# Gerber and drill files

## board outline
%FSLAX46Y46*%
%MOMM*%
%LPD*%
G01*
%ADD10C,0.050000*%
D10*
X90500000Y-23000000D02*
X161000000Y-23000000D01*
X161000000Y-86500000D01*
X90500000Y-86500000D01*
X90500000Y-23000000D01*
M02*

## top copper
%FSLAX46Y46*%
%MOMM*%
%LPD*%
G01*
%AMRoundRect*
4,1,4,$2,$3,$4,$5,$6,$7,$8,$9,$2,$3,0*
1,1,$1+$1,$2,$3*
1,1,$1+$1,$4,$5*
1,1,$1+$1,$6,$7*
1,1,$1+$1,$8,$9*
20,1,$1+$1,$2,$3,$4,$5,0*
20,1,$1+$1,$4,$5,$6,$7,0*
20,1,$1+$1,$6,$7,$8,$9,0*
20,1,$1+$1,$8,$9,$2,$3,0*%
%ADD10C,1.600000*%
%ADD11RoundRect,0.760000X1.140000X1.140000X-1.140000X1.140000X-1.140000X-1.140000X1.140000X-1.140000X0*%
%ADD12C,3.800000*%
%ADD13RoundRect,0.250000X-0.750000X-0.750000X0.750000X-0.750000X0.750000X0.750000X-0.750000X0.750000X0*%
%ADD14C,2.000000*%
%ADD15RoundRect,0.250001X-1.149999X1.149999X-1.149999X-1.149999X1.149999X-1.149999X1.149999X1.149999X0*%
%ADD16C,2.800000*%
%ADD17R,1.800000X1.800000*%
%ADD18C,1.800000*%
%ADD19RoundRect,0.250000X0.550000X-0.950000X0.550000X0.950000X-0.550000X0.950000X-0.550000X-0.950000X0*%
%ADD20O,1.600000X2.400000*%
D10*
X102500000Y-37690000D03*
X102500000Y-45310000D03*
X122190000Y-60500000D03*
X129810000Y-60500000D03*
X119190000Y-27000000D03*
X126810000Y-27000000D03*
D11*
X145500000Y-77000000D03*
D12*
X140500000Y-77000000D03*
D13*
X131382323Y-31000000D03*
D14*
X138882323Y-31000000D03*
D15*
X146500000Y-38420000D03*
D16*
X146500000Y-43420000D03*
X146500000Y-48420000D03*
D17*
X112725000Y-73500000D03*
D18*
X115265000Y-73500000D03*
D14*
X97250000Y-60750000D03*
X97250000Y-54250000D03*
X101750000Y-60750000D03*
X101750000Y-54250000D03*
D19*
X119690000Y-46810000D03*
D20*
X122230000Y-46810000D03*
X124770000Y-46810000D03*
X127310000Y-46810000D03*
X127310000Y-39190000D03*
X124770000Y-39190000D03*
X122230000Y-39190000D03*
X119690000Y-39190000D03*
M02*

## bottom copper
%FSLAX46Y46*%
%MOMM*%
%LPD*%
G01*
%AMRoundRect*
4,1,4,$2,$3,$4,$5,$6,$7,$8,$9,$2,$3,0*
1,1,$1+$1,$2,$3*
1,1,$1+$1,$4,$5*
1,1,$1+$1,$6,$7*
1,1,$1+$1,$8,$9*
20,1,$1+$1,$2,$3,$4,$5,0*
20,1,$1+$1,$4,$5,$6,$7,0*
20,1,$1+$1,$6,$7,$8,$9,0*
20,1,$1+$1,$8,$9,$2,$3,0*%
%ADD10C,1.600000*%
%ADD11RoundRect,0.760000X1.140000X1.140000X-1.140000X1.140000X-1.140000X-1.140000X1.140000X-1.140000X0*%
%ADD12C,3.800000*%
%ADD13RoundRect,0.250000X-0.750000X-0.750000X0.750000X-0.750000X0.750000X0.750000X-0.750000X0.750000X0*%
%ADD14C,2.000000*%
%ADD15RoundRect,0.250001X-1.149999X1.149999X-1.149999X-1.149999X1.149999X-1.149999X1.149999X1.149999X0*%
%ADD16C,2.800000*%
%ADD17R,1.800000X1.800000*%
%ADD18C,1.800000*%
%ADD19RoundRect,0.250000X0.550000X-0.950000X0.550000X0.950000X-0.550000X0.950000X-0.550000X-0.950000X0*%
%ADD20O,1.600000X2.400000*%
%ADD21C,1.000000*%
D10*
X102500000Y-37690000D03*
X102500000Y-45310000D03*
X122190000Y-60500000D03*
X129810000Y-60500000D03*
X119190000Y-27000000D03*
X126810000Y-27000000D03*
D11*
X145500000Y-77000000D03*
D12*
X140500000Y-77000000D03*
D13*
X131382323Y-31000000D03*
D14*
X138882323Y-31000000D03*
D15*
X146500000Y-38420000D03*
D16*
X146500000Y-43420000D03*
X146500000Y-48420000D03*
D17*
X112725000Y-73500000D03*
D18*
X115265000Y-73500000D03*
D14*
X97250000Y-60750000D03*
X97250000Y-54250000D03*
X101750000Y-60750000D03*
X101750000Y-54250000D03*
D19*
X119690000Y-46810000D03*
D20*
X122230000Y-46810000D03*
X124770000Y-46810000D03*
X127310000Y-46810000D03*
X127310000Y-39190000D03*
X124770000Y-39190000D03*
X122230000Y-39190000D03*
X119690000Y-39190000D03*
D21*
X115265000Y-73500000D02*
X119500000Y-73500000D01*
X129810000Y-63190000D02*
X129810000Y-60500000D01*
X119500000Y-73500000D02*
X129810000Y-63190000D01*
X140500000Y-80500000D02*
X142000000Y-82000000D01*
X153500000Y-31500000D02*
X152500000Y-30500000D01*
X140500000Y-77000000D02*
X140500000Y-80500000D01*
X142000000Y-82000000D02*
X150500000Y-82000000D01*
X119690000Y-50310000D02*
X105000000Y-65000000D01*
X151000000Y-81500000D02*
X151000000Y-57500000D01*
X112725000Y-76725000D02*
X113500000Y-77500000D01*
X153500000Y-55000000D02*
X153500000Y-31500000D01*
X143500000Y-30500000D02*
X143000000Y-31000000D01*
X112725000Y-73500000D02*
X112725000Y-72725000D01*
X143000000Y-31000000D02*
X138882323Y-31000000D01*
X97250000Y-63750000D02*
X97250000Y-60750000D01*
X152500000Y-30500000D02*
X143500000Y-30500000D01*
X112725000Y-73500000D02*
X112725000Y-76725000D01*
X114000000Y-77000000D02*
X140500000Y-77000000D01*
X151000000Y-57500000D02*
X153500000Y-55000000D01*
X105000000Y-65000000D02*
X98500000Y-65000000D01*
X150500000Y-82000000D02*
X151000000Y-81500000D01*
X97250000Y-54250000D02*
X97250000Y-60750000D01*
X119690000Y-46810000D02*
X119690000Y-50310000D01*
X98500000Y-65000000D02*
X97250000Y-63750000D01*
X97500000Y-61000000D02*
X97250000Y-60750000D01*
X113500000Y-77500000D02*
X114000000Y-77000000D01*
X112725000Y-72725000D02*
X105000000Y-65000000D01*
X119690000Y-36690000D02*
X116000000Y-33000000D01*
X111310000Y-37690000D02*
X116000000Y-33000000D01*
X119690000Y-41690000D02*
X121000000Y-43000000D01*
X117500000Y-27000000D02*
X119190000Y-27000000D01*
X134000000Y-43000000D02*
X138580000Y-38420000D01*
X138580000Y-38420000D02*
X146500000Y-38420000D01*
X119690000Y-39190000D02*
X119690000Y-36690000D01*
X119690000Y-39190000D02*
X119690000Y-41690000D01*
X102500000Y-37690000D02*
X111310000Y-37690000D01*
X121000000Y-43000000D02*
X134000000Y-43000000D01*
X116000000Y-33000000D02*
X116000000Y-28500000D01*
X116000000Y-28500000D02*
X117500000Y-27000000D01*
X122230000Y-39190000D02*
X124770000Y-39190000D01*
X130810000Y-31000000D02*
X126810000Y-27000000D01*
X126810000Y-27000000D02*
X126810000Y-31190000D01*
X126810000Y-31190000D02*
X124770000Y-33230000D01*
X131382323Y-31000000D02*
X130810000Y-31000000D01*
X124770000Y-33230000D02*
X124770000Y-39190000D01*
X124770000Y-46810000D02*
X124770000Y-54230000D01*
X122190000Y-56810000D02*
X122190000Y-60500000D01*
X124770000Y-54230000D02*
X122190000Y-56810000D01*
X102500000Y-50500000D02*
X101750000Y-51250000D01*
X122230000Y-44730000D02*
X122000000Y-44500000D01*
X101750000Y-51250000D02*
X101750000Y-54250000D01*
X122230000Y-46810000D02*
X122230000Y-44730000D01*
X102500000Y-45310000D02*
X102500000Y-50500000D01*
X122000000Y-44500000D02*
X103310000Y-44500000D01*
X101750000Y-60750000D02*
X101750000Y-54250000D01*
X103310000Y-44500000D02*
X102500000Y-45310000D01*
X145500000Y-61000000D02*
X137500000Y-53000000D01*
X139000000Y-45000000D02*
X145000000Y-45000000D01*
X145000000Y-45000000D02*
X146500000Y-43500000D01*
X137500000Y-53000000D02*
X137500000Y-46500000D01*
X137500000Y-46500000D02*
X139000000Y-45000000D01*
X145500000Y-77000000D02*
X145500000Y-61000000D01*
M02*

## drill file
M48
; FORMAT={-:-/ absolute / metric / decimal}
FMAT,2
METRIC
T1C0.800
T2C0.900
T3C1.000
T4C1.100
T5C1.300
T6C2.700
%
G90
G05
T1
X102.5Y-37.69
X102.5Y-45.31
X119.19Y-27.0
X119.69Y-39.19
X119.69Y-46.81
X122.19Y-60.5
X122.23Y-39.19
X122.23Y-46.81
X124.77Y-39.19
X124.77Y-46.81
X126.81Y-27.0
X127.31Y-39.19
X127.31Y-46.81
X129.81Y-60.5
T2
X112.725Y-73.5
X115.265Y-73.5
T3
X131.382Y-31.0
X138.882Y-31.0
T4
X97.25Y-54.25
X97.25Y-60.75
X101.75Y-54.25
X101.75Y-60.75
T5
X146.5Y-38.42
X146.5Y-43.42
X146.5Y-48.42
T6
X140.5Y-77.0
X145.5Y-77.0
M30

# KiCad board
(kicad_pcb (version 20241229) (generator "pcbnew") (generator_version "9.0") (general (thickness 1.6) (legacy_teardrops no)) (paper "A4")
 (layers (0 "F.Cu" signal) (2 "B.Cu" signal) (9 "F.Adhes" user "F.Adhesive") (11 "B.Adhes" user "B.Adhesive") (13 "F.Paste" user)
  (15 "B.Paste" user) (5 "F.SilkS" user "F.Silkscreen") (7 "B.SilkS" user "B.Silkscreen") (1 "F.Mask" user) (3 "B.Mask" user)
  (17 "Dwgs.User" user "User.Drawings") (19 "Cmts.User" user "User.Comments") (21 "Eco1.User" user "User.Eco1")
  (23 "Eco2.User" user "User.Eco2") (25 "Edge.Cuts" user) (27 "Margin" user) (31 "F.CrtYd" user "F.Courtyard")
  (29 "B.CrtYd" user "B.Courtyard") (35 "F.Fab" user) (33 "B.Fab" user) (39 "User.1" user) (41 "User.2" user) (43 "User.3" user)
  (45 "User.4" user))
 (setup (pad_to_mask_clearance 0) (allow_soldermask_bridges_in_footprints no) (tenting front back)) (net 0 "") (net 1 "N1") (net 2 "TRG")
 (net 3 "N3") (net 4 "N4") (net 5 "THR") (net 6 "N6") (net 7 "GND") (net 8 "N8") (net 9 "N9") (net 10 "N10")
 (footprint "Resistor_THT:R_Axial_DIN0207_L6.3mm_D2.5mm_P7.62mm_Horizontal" (layer "F.Cu") (at 102.5 37.69 -90)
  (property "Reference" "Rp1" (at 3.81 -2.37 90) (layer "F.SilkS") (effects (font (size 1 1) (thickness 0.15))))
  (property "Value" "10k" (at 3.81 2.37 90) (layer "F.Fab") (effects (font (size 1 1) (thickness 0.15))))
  (pad "1" thru_hole circle (at 0 0 270) (size 1.6 1.6) (drill 0.8) (layers "*.Cu" "*.Mask") (remove_unused_layers no) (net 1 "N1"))
  (pad "2" thru_hole circle (at 7.62 0 270) (size 1.6 1.6) (drill 0.8) (layers "*.Cu" "*.Mask") (remove_unused_layers no) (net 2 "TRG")))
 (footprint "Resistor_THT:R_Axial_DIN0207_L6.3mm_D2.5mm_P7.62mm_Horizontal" (layer "F.Cu") (at 122.19 60.5)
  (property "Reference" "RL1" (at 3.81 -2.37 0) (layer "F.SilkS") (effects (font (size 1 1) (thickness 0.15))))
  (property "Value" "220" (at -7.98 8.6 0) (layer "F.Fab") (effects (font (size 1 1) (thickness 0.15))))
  (pad "1" thru_hole circle (at 0 0) (size 1.6 1.6) (drill 0.8) (layers "*.Cu" "*.Mask") (remove_unused_layers no) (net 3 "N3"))
  (pad "2" thru_hole circle (at 7.62 0) (size 1.6 1.6) (drill 0.8) (layers "*.Cu" "*.Mask") (remove_unused_layers no) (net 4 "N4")))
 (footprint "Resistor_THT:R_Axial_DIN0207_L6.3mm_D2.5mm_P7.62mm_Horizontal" (layer "F.Cu") (at 119.19 27)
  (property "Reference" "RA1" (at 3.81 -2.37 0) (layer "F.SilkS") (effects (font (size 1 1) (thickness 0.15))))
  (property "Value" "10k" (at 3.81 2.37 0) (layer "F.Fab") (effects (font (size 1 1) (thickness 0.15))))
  (pad "1" thru_hole circle (at 0 0) (size 1.6 1.6) (drill 0.8) (layers "*.Cu" "*.Mask") (remove_unused_layers no) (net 1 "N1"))
  (pad "2" thru_hole circle (at 7.62 0) (size 1.6 1.6) (drill 0.8) (layers "*.Cu" "*.Mask") (remove_unused_layers no) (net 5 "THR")))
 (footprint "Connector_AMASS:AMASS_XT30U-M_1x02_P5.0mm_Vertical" (layer "F.Cu") (at 145.5 77 180)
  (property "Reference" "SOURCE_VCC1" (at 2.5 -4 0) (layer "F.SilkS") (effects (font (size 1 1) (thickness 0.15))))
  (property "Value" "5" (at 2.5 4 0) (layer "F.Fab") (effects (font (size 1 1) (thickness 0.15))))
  (pad "1" thru_hole roundrect (at 0 0 180) (size 3.8 3.8) (drill 2.7) (layers "*.Cu" "*.Mask") (remove_unused_layers no)
   (roundrect_rratio 0.2) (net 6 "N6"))
  (pad "2" thru_hole circle (at 5 0 180) (size 3.8 3.8) (drill 2.7) (layers "*.Cu" "*.Mask") (remove_unused_layers no) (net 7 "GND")))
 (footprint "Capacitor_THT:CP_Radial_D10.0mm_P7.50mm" (layer "F.Cu") (at 131.382323 31)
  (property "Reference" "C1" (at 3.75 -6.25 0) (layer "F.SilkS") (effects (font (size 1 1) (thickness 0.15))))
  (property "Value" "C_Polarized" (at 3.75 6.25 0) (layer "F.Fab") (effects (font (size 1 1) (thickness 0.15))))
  (pad "1" thru_hole roundrect (at 0 0) (size 2 2) (drill 1) (layers "*.Cu" "*.Mask") (remove_unused_layers no) (roundrect_rratio 0.125)
   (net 5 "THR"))
  (pad "2" thru_hole circle (at 7.5 0) (size 2 2) (drill 1) (layers "*.Cu" "*.Mask") (remove_unused_layers no) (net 7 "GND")))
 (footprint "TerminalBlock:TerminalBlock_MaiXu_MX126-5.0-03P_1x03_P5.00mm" (layer "F.Cu") (at 146.5 38.42 -90)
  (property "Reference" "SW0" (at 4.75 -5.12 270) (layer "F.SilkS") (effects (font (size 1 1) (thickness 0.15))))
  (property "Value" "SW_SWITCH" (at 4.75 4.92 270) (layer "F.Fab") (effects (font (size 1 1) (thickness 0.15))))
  (pad "1" thru_hole roundrect (at 0 0 270) (size 2.8 2.8) (drill 1.3) (layers "*.Cu" "*.Mask") (remove_unused_layers no)
   (roundrect_rratio 0.089286) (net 1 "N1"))
  (pad "2" thru_hole circle (at 5 0 270) (size 2.8 2.8) (drill 1.3) (layers "*.Cu" "*.Mask") (remove_unused_layers no) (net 6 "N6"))
  (pad "3" thru_hole circle (at 10 0 270) (size 2.8 2.8) (drill 1.3) (layers "*.Cu" "*.Mask") (remove_unused_layers no) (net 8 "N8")))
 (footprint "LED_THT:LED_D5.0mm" (layer "F.Cu") (at 112.725 73.5)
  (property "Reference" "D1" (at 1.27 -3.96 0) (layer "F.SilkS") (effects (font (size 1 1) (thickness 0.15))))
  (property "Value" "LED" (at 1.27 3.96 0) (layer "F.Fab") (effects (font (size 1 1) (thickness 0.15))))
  (pad "1" thru_hole rect (at 0 0) (size 1.8 1.8) (drill 0.9) (layers "*.Cu" "*.Mask") (remove_unused_layers no) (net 7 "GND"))
  (pad "2" thru_hole circle (at 2.54 0) (size 1.8 1.8) (drill 0.9) (layers "*.Cu" "*.Mask") (remove_unused_layers no) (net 4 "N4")))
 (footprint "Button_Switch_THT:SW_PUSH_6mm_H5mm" (layer "F.Cu") (at 97.25 60.75 90)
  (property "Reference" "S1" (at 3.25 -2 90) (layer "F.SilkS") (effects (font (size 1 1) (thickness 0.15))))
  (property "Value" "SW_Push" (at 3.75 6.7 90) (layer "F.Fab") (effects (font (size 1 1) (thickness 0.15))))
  (pad "1" thru_hole circle (at 0 0 180) (size 2 2) (drill 1.1) (layers "*.Cu" "*.Mask") (remove_unused_layers no) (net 7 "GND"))
  (pad "1" thru_hole circle (at 6.5 0 180) (size 2 2) (drill 1.1) (layers "*.Cu" "*.Mask") (remove_unused_layers no) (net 7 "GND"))
  (pad "2" thru_hole circle (at 0 4.5 180) (size 2 2) (drill 1.1) (layers "*.Cu" "*.Mask") (remove_unused_layers no) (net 2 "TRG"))
  (pad "2" thru_hole circle (at 6.5 4.5 180) (size 2 2) (drill 1.1) (layers "*.Cu" "*.Mask") (remove_unused_layers no) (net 2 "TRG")))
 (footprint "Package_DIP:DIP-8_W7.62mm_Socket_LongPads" (layer "F.Cu") (at 119.69 46.81 90)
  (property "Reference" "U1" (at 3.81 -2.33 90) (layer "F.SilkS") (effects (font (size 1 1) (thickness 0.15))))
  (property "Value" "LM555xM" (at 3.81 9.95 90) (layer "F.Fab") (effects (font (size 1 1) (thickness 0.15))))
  (pad "1" thru_hole roundrect (at 0 0 90) (size 2.4 1.6) (drill 0.8) (layers "*.Cu" "*.Mask") (remove_unused_layers no)
   (roundrect_rratio 0.15625) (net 7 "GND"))
  (pad "2" thru_hole oval (at 0 2.54 90) (size 2.4 1.6) (drill 0.8) (layers "*.Cu" "*.Mask") (remove_unused_layers no) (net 2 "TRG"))
  (pad "3" thru_hole oval (at 0 5.08 90) (size 2.4 1.6) (drill 0.8) (layers "*.Cu" "*.Mask") (remove_unused_layers no) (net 3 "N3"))
  (pad "4" thru_hole oval (at 0 7.62 90) (size 2.4 1.6) (drill 0.8) (layers "*.Cu" "*.Mask") (remove_unused_layers no) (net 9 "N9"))
  (pad "5" thru_hole oval (at 7.62 7.62 90) (size 2.4 1.6) (drill 0.8) (layers "*.Cu" "*.Mask") (remove_unused_layers no) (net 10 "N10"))
  (pad "6" thru_hole oval (at 7.62 5.08 90) (size 2.4 1.6) (drill 0.8) (layers "*.Cu" "*.Mask") (remove_unused_layers no) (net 5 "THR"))
  (pad "7" thru_hole oval (at 7.62 2.54 90) (size 2.4 1.6) (drill 0.8) (layers "*.Cu" "*.Mask") (remove_unused_layers no) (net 5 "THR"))
  (pad "8" thru_hole oval (at 7.62 0 90) (size 2.4 1.6) (drill 0.8) (layers "*.Cu" "*.Mask") (remove_unused_layers no) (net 1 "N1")))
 (gr_rect (start 90.5 23) (end 161 86.5) (stroke (width 0.05) (type default)) (fill no) (layer "Edge.Cuts"))
 (segment (start 115.265 73.5) (end 119.5 73.5) (width 1) (layer "B.Cu") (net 4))
 (segment (start 129.81 63.19) (end 129.81 60.5) (width 1) (layer "B.Cu") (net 4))
 (segment (start 119.5 73.5) (end 129.81 63.19) (width 1) (layer "B.Cu") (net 4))
 (segment (start 140.5 80.5) (end 142 82) (width 1) (layer "B.Cu") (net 7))
 (segment (start 153.5 31.5) (end 152.5 30.5) (width 1) (layer "B.Cu") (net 7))
 (segment (start 140.5 77) (end 140.5 80.5) (width 1) (layer "B.Cu") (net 7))
 (segment (start 142 82) (end 150.5 82) (width 1) (layer "B.Cu") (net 7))
 (segment (start 119.69 50.31) (end 105 65) (width 1) (layer "B.Cu") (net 7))
 (segment (start 151 81.5) (end 151 57.5) (width 1) (layer "B.Cu") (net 7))
 (segment (start 112.725 76.725) (end 113.5 77.5) (width 1) (layer "B.Cu") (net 7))
 (segment (start 153.5 55) (end 153.5 31.5) (width 1) (layer "B.Cu") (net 7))
 (segment (start 143.5 30.5) (end 143 31) (width 1) (layer "B.Cu") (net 7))
 (segment (start 112.725 73.5) (end 112.725 72.725) (width 1) (layer "B.Cu") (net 7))
 (segment (start 143 31) (end 138.882323 31) (width 1) (layer "B.Cu") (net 7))
 (segment (start 97.25 63.75) (end 97.25 60.75) (width 1) (layer "B.Cu") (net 7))
 (segment (start 152.5 30.5) (end 143.5 30.5) (width 1) (layer "B.Cu") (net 7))
 (segment (start 112.725 73.5) (end 112.725 76.725) (width 1) (layer "B.Cu") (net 7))
 (segment (start 114 77) (end 140.5 77) (width 1) (layer "B.Cu") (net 7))
 (segment (start 151 57.5) (end 153.5 55) (width 1) (layer "B.Cu") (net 7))
 (segment (start 105 65) (end 98.5 65) (width 1) (layer "B.Cu") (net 7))
 (segment (start 150.5 82) (end 151 81.5) (width 1) (layer "B.Cu") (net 7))
 (segment (start 97.25 54.25) (end 97.25 60.75) (width 1) (layer "B.Cu") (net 7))
 (segment (start 119.69 46.81) (end 119.69 50.31) (width 1) (layer "B.Cu") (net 7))
 (segment (start 98.5 65) (end 97.25 63.75) (width 1) (layer "B.Cu") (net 7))
 (segment (start 97.5 61) (end 97.25 60.75) (width 1) (layer "B.Cu") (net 7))
 (segment (start 113.5 77.5) (end 114 77) (width 1) (layer "B.Cu") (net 7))
 (segment (start 112.725 72.725) (end 105 65) (width 1) (layer "B.Cu") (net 7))
 (segment (start 119.69 36.69) (end 116 33) (width 1) (layer "B.Cu") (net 1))
 (segment (start 111.31 37.69) (end 116 33) (width 1) (layer "B.Cu") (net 1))
 (segment (start 119.69 41.69) (end 121 43) (width 1) (layer "B.Cu") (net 1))
 (segment (start 117.5 27) (end 119.19 27) (width 1) (layer "B.Cu") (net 1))
 (segment (start 134 43) (end 138.58 38.42) (width 1) (layer "B.Cu") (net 1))
 (segment (start 138.58 38.42) (end 146.5 38.42) (width 1) (layer "B.Cu") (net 1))
 (segment (start 119.69 39.19) (end 119.69 36.69) (width 1) (layer "B.Cu") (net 1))
 (segment (start 119.69 39.19) (end 119.69 41.69) (width 1) (layer "B.Cu") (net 1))
 (segment (start 102.5 37.69) (end 111.31 37.69) (width 1) (layer "B.Cu") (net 1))
 (segment (start 121 43) (end 134 43) (width 1) (layer "B.Cu") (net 1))
 (segment (start 116 33) (end 116 28.5) (width 1) (layer "B.Cu") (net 1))
 (segment (start 116 28.5) (end 117.5 27) (width 1) (layer "B.Cu") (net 1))
 (segment (start 122.23 39.19) (end 124.77 39.19) (width 1) (layer "B.Cu") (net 5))
 (segment (start 130.81 31) (end 126.81 27) (width 1) (layer "B.Cu") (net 5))
 (segment (start 126.81 27) (end 126.81 31.19) (width 1) (layer "B.Cu") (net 5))
 (segment (start 126.81 31.19) (end 124.77 33.23) (width 1) (layer "B.Cu") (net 5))
 (segment (start 131.382323 31) (end 130.81 31) (width 1) (layer "B.Cu") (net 5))
 (segment (start 124.77 33.23) (end 124.77 39.19) (width 1) (layer "B.Cu") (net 5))
 (segment (start 124.77 46.81) (end 124.77 54.23) (width 1) (layer "B.Cu") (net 3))
 (segment (start 122.19 56.81) (end 122.19 60.5) (width 1) (layer "B.Cu") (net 3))
 (segment (start 124.77 54.23) (end 122.19 56.81) (width 1) (layer "B.Cu") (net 3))
 (segment (start 102.5 50.5) (end 101.75 51.25) (width 1) (layer "B.Cu") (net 2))
 (segment (start 122.23 44.73) (end 122 44.5) (width 1) (layer "B.Cu") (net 2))
 (segment (start 101.75 51.25) (end 101.75 54.25) (width 1) (layer "B.Cu") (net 2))
 (segment (start 122.23 46.81) (end 122.23 44.73) (width 1) (layer "B.Cu") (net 2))
 (segment (start 102.5 45.31) (end 102.5 50.5) (width 1) (layer "B.Cu") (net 2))
 (segment (start 122 44.5) (end 103.31 44.5) (width 1) (layer "B.Cu") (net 2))
 (segment (start 101.75 60.75) (end 101.75 54.25) (width 1) (layer "B.Cu") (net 2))
 (segment (start 103.31 44.5) (end 102.5 45.31) (width 1) (layer "B.Cu") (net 2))
 (segment (start 145.5 61) (end 137.5 53) (width 1) (layer "B.Cu") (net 6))
 (segment (start 139 45) (end 145 45) (width 1) (layer "B.Cu") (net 6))
 (segment (start 145 45) (end 146.5 43.5) (width 1) (layer "B.Cu") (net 6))
 (segment (start 137.5 53) (end 137.5 46.5) (width 1) (layer "B.Cu") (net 6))
 (segment (start 137.5 46.5) (end 139 45) (width 1) (layer "B.Cu") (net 6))
 (segment (start 145.5 77) (end 145.5 61) (width 1) (layer "B.Cu") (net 6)))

